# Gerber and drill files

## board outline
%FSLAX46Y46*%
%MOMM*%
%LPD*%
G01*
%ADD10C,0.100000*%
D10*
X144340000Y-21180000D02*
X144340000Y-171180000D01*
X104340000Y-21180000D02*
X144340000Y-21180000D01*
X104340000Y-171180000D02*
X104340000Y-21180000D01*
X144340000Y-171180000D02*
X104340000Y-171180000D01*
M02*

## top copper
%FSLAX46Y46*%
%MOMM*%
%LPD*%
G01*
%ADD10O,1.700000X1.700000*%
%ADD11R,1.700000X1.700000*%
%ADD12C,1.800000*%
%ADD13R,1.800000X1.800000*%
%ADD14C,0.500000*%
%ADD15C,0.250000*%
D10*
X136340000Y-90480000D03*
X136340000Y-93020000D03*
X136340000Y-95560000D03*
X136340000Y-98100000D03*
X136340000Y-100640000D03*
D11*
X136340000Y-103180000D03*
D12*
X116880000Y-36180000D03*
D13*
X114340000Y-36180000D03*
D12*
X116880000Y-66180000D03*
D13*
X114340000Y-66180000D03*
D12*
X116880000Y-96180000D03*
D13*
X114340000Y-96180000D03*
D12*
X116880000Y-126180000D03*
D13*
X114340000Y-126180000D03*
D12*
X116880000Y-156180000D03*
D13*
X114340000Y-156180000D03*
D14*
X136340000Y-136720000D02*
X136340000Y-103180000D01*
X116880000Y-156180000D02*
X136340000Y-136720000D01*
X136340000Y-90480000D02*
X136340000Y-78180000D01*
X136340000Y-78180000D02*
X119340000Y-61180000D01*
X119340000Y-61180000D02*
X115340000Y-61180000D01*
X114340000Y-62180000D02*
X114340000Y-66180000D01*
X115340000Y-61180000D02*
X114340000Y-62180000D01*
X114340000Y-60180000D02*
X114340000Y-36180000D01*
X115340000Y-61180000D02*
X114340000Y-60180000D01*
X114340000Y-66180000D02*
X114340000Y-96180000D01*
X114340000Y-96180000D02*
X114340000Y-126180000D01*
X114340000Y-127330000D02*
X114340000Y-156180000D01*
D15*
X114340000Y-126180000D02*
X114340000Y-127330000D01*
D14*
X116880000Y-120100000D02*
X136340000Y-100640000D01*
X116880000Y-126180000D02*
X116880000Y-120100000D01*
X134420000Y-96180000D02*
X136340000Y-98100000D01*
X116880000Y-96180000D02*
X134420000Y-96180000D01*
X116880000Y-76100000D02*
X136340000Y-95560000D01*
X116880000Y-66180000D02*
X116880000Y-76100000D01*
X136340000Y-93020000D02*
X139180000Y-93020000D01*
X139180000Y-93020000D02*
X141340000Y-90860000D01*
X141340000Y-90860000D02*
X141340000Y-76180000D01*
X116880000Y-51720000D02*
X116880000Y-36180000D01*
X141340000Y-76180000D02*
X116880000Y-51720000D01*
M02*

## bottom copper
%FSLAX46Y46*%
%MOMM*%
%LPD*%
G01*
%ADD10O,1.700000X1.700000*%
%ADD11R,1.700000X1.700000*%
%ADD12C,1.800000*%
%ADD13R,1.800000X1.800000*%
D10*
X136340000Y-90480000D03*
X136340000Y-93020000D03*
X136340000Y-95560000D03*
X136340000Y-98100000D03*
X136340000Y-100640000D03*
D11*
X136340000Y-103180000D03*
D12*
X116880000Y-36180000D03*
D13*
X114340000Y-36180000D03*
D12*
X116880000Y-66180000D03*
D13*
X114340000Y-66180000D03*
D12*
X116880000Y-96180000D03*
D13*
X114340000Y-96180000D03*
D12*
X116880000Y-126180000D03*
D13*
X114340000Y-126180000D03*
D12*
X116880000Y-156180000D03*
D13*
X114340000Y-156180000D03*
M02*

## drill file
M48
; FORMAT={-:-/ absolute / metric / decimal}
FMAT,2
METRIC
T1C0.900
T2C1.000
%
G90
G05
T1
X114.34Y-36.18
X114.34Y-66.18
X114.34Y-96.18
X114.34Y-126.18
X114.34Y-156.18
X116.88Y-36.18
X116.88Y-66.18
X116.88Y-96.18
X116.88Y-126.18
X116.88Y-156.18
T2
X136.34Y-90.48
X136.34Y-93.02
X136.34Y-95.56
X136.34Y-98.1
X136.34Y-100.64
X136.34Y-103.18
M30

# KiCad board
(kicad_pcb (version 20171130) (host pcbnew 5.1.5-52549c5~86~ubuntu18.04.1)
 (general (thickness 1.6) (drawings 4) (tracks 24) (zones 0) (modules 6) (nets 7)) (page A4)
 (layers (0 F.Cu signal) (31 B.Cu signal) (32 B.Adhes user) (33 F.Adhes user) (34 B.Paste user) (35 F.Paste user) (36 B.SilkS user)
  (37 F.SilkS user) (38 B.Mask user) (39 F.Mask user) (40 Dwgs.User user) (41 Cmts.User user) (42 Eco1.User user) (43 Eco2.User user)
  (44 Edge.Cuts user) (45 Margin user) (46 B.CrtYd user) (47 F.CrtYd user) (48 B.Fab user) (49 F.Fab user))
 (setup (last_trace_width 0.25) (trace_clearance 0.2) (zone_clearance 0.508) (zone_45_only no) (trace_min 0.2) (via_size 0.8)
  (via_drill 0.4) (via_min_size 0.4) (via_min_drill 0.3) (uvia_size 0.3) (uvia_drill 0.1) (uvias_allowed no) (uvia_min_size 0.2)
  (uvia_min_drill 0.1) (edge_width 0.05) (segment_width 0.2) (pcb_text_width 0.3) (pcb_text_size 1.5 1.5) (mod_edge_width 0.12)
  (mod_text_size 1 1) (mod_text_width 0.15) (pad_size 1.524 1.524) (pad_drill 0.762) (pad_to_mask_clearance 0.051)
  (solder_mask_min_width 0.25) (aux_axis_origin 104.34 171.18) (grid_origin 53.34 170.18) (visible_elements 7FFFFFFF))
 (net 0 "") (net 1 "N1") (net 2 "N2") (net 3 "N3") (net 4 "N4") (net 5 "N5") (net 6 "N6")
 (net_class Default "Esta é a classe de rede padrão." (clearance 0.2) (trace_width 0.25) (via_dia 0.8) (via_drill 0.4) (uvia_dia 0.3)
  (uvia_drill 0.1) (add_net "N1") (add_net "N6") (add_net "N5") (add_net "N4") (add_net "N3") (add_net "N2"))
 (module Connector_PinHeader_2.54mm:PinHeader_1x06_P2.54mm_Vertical (layer F.Cu) (at 136.34 103.18 180)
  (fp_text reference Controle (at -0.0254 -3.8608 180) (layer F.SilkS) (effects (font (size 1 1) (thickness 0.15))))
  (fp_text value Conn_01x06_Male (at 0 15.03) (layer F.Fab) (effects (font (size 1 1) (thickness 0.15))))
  (pad 6 thru_hole oval (at 0 12.7 180) (size 1.7 1.7) (drill 1) (layers *.Cu *.Mask) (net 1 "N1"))
  (pad 5 thru_hole oval (at 0 10.16 180) (size 1.7 1.7) (drill 1) (layers *.Cu *.Mask) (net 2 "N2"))
  (pad 4 thru_hole oval (at 0 7.62 180) (size 1.7 1.7) (drill 1) (layers *.Cu *.Mask) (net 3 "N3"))
  (pad 3 thru_hole oval (at 0 5.08 180) (size 1.7 1.7) (drill 1) (layers *.Cu *.Mask) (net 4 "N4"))
  (pad 2 thru_hole oval (at 0 2.54 180) (size 1.7 1.7) (drill 1) (layers *.Cu *.Mask) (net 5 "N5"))
  (pad 1 thru_hole rect (at 0 0 180) (size 1.7 1.7) (drill 1) (layers *.Cu *.Mask) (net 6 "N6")))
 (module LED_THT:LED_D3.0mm (layer F.Cu) (at 114.34 36.18)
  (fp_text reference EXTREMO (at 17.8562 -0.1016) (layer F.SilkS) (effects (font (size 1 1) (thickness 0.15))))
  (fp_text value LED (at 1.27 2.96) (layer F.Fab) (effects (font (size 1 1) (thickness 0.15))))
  (pad 2 thru_hole circle (at 2.54 0) (size 1.8 1.8) (drill 0.9) (layers *.Cu *.Mask) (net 2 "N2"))
  (pad 1 thru_hole rect (at 0 0) (size 1.8 1.8) (drill 0.9) (layers *.Cu *.Mask) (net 1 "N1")))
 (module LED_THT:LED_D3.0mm (layer F.Cu) (at 114.34 66.18)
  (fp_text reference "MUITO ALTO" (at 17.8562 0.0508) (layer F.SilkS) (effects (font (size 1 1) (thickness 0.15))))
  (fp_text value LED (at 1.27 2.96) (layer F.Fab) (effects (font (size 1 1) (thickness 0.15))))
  (pad 2 thru_hole circle (at 2.54 0) (size 1.8 1.8) (drill 0.9) (layers *.Cu *.Mask) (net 3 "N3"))
  (pad 1 thru_hole rect (at 0 0) (size 1.8 1.8) (drill 0.9) (layers *.Cu *.Mask) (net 1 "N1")))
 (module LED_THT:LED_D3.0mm (layer F.Cu) (at 114.34 96.18)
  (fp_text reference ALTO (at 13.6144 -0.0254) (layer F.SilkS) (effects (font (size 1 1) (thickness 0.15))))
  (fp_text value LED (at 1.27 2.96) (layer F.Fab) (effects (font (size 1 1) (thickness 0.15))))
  (pad 2 thru_hole circle (at 2.54 0) (size 1.8 1.8) (drill 0.9) (layers *.Cu *.Mask) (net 4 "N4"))
  (pad 1 thru_hole rect (at 0 0) (size 1.8 1.8) (drill 0.9) (layers *.Cu *.Mask) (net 1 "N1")))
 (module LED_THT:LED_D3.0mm (layer F.Cu) (at 114.34 126.18)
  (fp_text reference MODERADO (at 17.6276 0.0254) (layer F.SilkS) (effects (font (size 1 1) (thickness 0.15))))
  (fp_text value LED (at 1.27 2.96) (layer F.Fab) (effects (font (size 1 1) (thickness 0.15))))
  (pad 2 thru_hole circle (at 2.54 0) (size 1.8 1.8) (drill 0.9) (layers *.Cu *.Mask) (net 5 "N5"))
  (pad 1 thru_hole rect (at 0 0) (size 1.8 1.8) (drill 0.9) (layers *.Cu *.Mask) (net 1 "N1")))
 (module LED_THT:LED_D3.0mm (layer F.Cu) (at 114.34 156.18)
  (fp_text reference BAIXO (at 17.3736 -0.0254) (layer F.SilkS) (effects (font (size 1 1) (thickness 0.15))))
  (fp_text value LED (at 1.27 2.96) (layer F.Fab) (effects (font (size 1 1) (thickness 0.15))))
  (pad 2 thru_hole circle (at 2.54 0) (size 1.8 1.8) (drill 0.9) (layers *.Cu *.Mask) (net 6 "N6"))
  (pad 1 thru_hole rect (at 0 0) (size 1.8 1.8) (drill 0.9) (layers *.Cu *.Mask) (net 1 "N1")))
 (gr_line (start 144.34 21.18) (end 144.34 171.18) (layer Edge.Cuts) (width 0.1))
 (gr_line (start 104.34 21.18) (end 144.34 21.18) (layer Edge.Cuts) (width 0.1))
 (gr_line (start 104.34 171.18) (end 104.34 21.18) (layer Edge.Cuts) (width 0.1))
 (gr_line (start 144.34 171.18) (end 104.34 171.18) (layer Edge.Cuts) (width 0.1))
 (segment (start 136.34 136.72) (end 136.34 103.18) (width 0.5) (layer F.Cu) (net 6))
 (segment (start 116.88 156.18) (end 136.34 136.72) (width 0.5) (layer F.Cu) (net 6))
 (segment (start 136.34 90.48) (end 136.34 78.18) (width 0.5) (layer F.Cu) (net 1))
 (segment (start 136.34 78.18) (end 119.34 61.18) (width 0.5) (layer F.Cu) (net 1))
 (segment (start 119.34 61.18) (end 115.34 61.18) (width 0.5) (layer F.Cu) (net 1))
 (segment (start 114.34 62.18) (end 114.34 66.18) (width 0.5) (layer F.Cu) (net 1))
 (segment (start 115.34 61.18) (end 114.34 62.18) (width 0.5) (layer F.Cu) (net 1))
 (segment (start 114.34 60.18) (end 114.34 36.18) (width 0.5) (layer F.Cu) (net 1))
 (segment (start 115.34 61.18) (end 114.34 60.18) (width 0.5) (layer F.Cu) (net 1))
 (segment (start 114.34 66.18) (end 114.34 96.18) (width 0.5) (layer F.Cu) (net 1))
 (segment (start 114.34 96.18) (end 114.34 126.18) (width 0.5) (layer F.Cu) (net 1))
 (segment (start 114.34 127.33) (end 114.34 156.18) (width 0.5) (layer F.Cu) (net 1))
 (segment (start 114.34 126.18) (end 114.34 127.33) (width 0.25) (layer F.Cu) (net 1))
 (segment (start 116.88 120.1) (end 136.34 100.64) (width 0.5) (layer F.Cu) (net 5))
 (segment (start 116.88 126.18) (end 116.88 120.1) (width 0.5) (layer F.Cu) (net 5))
 (segment (start 134.42 96.18) (end 136.34 98.1) (width 0.5) (layer F.Cu) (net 4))
 (segment (start 116.88 96.18) (end 134.42 96.18) (width 0.5) (layer F.Cu) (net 4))
 (segment (start 116.88 76.1) (end 136.34 95.56) (width 0.5) (layer F.Cu) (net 3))
 (segment (start 116.88 66.18) (end 116.88 76.1) (width 0.5) (layer F.Cu) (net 3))
 (segment (start 136.34 93.02) (end 139.18 93.02) (width 0.5) (layer F.Cu) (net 2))
 (segment (start 139.18 93.02) (end 141.34 90.86) (width 0.5) (layer F.Cu) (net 2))
 (segment (start 141.34 90.86) (end 141.34 76.18) (width 0.5) (layer F.Cu) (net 2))
 (segment (start 116.88 51.72) (end 116.88 36.18) (width 0.5) (layer F.Cu) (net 2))
 (segment (start 141.34 76.18) (end 116.88 51.72) (width 0.5) (layer F.Cu) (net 2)))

